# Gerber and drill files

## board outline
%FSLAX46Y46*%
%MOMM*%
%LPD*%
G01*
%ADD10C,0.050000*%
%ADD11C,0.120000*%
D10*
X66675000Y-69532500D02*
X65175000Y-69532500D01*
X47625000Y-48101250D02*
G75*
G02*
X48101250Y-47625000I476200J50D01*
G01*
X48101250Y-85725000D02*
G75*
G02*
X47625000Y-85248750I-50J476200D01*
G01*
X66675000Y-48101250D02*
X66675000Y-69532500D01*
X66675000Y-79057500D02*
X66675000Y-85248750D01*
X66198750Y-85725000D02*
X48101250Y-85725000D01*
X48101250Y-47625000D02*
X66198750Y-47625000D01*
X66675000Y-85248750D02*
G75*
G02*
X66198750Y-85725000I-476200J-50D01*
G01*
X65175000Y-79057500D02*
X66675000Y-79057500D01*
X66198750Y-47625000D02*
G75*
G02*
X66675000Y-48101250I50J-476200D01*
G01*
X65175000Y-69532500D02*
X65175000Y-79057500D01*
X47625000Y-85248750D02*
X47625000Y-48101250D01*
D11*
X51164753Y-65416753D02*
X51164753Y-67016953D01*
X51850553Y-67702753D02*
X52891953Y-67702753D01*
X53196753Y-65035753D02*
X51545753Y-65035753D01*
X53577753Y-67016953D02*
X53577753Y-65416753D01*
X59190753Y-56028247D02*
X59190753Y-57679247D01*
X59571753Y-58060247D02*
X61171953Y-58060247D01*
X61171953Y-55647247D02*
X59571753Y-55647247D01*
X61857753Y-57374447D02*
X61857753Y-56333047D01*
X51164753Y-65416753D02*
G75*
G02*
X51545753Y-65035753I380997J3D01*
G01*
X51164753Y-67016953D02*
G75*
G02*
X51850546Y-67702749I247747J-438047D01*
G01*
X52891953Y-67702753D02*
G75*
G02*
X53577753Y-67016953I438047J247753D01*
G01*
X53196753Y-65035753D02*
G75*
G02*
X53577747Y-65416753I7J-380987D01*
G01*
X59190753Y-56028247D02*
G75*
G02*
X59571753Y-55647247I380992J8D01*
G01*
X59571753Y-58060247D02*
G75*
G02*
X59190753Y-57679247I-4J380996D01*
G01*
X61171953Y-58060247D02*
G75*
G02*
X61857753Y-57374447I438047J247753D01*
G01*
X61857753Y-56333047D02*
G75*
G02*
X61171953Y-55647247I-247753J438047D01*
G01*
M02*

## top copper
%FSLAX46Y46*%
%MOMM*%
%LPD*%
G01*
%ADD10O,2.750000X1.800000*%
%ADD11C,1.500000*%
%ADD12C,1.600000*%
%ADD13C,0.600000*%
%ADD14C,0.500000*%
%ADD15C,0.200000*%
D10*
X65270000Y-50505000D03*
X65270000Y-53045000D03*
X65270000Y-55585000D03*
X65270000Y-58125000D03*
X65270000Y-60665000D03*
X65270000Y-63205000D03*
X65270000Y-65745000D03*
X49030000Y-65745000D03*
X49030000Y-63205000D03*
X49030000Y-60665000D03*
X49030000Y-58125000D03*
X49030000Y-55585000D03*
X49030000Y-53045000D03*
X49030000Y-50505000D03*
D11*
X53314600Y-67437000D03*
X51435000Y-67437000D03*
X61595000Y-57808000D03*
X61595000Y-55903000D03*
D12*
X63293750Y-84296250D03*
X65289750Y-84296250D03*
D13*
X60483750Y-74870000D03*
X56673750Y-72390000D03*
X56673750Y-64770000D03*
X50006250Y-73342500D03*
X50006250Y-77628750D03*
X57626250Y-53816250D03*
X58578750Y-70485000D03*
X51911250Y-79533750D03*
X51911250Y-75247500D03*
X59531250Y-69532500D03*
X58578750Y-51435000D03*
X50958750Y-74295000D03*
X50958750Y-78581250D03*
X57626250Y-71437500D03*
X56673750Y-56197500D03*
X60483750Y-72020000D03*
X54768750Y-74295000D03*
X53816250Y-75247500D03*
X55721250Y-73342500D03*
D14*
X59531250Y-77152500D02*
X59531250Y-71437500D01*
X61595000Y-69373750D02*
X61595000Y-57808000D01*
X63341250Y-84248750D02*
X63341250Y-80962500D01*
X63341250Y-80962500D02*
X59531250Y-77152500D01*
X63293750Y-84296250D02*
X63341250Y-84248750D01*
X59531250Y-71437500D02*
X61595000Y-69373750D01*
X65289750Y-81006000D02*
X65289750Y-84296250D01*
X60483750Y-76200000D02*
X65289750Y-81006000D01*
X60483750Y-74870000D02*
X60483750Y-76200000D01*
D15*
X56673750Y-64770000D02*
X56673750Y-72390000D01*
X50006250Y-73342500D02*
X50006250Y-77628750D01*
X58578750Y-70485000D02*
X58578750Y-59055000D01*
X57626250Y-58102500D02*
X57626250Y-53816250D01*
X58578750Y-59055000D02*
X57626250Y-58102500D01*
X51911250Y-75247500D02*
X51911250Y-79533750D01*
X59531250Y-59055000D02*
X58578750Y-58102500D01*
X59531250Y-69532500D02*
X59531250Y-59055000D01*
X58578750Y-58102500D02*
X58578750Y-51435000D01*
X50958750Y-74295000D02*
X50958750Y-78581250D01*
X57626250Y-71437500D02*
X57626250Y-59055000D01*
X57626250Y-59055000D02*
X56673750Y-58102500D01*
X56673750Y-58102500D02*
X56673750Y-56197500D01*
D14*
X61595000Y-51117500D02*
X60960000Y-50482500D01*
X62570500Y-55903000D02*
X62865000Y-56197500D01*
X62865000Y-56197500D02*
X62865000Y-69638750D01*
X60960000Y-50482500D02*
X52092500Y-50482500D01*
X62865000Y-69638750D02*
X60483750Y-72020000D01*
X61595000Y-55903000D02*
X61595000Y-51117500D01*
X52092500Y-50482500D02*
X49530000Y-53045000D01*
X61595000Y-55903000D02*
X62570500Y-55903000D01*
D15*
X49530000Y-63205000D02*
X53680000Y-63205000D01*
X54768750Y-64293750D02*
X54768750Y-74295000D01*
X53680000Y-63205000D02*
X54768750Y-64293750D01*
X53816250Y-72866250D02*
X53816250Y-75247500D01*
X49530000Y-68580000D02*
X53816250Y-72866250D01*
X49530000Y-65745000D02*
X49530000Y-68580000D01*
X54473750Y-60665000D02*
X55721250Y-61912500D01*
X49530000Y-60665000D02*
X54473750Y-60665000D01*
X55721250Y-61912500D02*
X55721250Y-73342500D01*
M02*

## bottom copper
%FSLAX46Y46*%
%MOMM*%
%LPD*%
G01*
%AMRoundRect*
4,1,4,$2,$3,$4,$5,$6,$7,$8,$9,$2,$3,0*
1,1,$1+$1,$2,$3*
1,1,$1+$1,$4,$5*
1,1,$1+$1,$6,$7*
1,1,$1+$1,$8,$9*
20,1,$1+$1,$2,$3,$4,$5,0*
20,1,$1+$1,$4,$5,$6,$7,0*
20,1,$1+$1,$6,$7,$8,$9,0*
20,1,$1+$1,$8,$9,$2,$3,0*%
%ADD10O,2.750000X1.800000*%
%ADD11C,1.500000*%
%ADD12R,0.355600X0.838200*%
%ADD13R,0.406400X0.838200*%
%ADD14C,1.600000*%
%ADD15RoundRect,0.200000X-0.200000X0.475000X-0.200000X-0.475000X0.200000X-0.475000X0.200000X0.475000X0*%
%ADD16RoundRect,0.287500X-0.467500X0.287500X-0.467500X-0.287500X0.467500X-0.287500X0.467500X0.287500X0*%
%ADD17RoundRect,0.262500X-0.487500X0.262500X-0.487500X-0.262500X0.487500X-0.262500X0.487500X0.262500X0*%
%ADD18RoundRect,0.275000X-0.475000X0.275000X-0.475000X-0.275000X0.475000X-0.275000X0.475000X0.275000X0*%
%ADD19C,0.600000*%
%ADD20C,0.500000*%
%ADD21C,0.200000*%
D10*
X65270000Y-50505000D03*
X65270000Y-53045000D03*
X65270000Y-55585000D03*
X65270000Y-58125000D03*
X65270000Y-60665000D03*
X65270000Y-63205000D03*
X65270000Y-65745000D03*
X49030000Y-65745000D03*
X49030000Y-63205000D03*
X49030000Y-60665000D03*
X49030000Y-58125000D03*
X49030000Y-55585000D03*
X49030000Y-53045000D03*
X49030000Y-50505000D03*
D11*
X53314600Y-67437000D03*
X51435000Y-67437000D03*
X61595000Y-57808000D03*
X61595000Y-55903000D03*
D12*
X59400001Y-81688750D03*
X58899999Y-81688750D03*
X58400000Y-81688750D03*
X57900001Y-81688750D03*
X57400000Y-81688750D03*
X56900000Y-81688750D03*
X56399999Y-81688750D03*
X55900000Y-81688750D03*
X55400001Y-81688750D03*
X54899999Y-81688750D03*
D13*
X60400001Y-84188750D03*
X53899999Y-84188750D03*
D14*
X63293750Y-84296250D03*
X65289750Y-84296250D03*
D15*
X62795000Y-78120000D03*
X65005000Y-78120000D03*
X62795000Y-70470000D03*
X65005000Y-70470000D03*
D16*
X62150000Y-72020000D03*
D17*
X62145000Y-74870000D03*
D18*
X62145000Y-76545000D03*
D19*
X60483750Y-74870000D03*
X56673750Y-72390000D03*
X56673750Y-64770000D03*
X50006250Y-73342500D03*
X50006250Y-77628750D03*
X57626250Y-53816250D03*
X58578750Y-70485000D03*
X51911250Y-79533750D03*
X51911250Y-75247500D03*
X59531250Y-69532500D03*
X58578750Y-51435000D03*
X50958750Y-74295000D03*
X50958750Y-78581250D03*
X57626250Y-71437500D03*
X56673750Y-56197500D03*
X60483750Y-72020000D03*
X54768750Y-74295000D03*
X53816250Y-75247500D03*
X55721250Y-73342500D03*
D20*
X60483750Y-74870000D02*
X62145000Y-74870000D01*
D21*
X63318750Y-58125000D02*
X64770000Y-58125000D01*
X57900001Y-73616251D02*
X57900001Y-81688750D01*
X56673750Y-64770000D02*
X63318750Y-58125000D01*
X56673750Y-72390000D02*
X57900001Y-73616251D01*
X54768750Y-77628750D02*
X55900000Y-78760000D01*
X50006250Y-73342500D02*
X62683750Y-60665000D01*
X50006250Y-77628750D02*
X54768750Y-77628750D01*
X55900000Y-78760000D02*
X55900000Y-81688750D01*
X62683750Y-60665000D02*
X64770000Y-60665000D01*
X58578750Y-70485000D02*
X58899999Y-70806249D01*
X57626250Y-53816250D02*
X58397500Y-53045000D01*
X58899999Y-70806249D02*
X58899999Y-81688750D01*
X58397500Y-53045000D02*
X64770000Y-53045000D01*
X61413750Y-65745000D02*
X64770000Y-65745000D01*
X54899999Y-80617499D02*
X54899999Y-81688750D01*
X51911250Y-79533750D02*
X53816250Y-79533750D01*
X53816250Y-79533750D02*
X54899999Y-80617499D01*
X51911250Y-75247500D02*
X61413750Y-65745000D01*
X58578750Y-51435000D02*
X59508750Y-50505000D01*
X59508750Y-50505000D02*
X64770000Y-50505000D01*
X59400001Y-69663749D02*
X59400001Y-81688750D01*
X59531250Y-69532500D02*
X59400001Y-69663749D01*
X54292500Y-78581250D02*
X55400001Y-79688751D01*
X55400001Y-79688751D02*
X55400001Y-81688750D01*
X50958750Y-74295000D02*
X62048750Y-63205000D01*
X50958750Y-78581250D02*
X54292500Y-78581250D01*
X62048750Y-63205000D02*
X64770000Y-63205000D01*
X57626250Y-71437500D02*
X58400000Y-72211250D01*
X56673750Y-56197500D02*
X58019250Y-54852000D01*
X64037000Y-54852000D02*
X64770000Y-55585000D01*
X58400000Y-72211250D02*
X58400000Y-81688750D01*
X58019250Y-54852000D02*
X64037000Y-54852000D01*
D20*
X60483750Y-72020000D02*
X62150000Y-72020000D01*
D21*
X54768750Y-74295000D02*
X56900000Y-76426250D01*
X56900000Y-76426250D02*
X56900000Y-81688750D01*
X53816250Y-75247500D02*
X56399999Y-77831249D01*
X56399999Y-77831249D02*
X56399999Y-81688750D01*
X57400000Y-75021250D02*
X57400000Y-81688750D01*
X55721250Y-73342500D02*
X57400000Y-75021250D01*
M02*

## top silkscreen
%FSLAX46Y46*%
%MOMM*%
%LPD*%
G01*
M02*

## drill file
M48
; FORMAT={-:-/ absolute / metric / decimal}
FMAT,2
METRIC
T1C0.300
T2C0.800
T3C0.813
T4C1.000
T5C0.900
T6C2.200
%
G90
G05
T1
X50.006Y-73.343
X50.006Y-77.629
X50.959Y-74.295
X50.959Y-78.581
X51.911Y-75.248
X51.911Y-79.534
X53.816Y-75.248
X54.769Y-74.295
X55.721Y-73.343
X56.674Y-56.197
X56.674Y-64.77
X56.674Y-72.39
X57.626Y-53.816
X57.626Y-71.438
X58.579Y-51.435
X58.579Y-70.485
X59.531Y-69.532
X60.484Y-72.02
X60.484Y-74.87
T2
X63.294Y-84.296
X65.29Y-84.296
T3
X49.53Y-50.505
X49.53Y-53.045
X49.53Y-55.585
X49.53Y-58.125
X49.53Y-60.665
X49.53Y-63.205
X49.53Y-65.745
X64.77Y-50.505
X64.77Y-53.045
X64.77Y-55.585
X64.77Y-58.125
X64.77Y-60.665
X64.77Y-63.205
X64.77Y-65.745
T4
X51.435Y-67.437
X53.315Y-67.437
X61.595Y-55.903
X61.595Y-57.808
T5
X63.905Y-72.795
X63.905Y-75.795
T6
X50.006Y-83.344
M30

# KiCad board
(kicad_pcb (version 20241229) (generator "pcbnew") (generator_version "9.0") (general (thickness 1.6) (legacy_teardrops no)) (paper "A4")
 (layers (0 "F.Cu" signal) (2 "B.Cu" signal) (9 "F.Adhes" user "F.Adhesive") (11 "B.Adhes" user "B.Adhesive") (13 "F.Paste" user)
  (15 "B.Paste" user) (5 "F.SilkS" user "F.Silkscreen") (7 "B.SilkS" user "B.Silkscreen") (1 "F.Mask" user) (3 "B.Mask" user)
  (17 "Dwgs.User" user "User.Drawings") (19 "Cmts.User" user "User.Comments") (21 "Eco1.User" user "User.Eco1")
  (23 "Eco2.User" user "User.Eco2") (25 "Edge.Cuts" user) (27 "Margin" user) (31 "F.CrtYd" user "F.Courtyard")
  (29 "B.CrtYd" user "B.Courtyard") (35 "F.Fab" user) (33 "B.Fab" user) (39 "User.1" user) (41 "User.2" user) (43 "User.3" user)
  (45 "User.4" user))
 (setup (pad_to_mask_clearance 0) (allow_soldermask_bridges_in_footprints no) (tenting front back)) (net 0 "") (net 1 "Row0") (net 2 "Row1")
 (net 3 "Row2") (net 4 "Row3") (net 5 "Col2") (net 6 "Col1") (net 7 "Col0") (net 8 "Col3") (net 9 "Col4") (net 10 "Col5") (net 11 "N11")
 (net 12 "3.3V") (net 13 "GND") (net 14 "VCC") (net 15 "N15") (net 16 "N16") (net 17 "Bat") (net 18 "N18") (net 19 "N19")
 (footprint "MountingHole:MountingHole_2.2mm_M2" (layer "F.Cu") (at 50.00625 83.34375)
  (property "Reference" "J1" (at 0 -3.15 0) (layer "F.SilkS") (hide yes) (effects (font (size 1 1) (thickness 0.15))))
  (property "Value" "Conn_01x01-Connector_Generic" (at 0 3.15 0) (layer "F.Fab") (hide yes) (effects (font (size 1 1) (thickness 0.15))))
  (pad "" np_thru_hole circle (at 0 0) (size 2.2 2.2) (drill 2.2) (layers "*.Cu" "*.Mask")))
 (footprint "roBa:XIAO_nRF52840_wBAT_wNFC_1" (layer "B.Cu") (at 57.15 47.625 180)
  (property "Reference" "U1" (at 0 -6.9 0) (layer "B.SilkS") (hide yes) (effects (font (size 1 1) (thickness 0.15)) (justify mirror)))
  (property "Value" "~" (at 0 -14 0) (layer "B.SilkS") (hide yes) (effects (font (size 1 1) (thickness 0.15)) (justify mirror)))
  (fp_line (start 5.985247 -17.791753) (end 5.985247 -19.391953) (stroke (width 0.12) (type solid)) (layer "Edge.Cuts"))
  (fp_line (start 5.299447 -20.077753) (end 4.258047 -20.077753) (stroke (width 0.12) (type solid)) (layer "Edge.Cuts"))
  (fp_line (start 3.953247 -17.410753) (end 5.604247 -17.410753) (stroke (width 0.12) (type solid)) (layer "Edge.Cuts"))
  (fp_line (start 3.572247 -19.391953) (end 3.572247 -17.791753) (stroke (width 0.12) (type solid)) (layer "Edge.Cuts"))
  (fp_line (start -2.040753 -8.403247) (end -2.040753 -10.054247) (stroke (width 0.12) (type solid)) (layer "Edge.Cuts"))
  (fp_line (start -2.421753 -10.435247) (end -4.021953 -10.435247) (stroke (width 0.12) (type solid)) (layer "Edge.Cuts"))
  (fp_line (start -4.021953 -8.022247) (end -2.421753 -8.022247) (stroke (width 0.12) (type solid)) (layer "Edge.Cuts"))
  (fp_line (start -4.707753 -9.749447) (end -4.707753 -8.708047) (stroke (width 0.12) (type solid)) (layer "Edge.Cuts"))
  (fp_arc (start 5.985247 -17.791753) (mid 5.873656 -17.522344) (end 5.604247 -17.410753) (stroke (width 0.12) (type solid))
   (layer "Edge.Cuts"))
  (fp_arc (start 5.985247 -19.391953) (mid 5.381645 -19.474147) (end 5.299447 -20.077753) (stroke (width 0.12) (type solid))
   (layer "Edge.Cuts"))
  (fp_arc (start 4.258047 -20.077753) (mid 4.175856 -19.474144) (end 3.572247 -19.391953) (stroke (width 0.12) (type solid))
   (layer "Edge.Cuts"))
  (fp_arc (start 3.953247 -17.410753) (mid 3.683836 -17.522343) (end 3.572247 -17.791753) (stroke (width 0.12) (type solid))
   (layer "Edge.Cuts"))
  (fp_arc (start -2.040753 -8.403247) (mid -2.152343 -8.133837) (end -2.421753 -8.022247) (stroke (width 0.12) (type solid))
   (layer "Edge.Cuts"))
  (fp_arc (start -2.421753 -10.435247) (mid -2.152344 -10.323656) (end -2.040753 -10.054247) (stroke (width 0.12) (type solid))
   (layer "Edge.Cuts"))
  (fp_arc (start -4.021953 -10.435247) (mid -4.104144 -9.831638) (end -4.707753 -9.749447) (stroke (width 0.12) (type solid))
   (layer "Edge.Cuts"))
  (fp_arc (start -4.707753 -8.708047) (mid -4.104144 -8.625856) (end -4.021953 -8.022247) (stroke (width 0.12) (type solid))
   (layer "Edge.Cuts"))
  (pad "1" thru_hole oval (at -7.62 -2.88 180) (size 2.75 1.8) (drill 0.8128 (offset -0.5 0)) (layers "*.Cu" "*.Mask")
   (remove_unused_layers no) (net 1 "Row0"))
  (pad "2" thru_hole oval (at -7.62 -5.42 180) (size 2.75 1.8) (drill 0.8128 (offset -0.5 0)) (layers "*.Cu" "*.Mask")
   (remove_unused_layers no) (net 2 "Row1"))
  (pad "3" thru_hole oval (at -7.62 -7.96 180) (size 2.75 1.8) (drill 0.8128 (offset -0.5 0)) (layers "*.Cu" "*.Mask")
   (remove_unused_layers no) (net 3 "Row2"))
  (pad "4" thru_hole oval (at -7.62 -10.5 180) (size 2.75 1.8) (drill 0.8128 (offset -0.5 0)) (layers "*.Cu" "*.Mask")
   (remove_unused_layers no) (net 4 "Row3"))
  (pad "5" thru_hole oval (at -7.62 -13.04 180) (size 2.75 1.8) (drill 0.8128 (offset -0.5 0)) (layers "*.Cu" "*.Mask")
   (remove_unused_layers no) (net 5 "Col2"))
  (pad "6" thru_hole oval (at -7.62 -15.58 180) (size 2.75 1.8) (drill 0.8128 (offset -0.5 0)) (layers "*.Cu" "*.Mask")
   (remove_unused_layers no) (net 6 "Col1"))
  (pad "7" thru_hole oval (at -7.62 -18.12 180) (size 2.75 1.8) (drill 0.8128 (offset -0.5 0)) (layers "*.Cu" "*.Mask")
   (remove_unused_layers no) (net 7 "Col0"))
  (pad "8" thru_hole oval (at 7.62 -18.12 180) (size 2.75 1.8) (drill 0.8128 (offset 0.5 0)) (layers "*.Cu" "*.Mask")
   (remove_unused_layers no) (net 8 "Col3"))
  (pad "9" thru_hole oval (at 7.62 -15.58 180) (size 2.75 1.8) (drill 0.8128 (offset 0.5 0)) (layers "*.Cu" "*.Mask")
   (remove_unused_layers no) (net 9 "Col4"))
  (pad "10" thru_hole oval (at 7.62 -13.04 180) (size 2.75 1.8) (drill 0.8128 (offset 0.5 0)) (layers "*.Cu" "*.Mask")
   (remove_unused_layers no) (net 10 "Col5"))
  (pad "11" thru_hole oval (at 7.62 -10.5 180) (size 2.75 1.8) (drill 0.8128 (offset 0.5 0)) (layers "*.Cu" "*.Mask")
   (remove_unused_layers no) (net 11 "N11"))
  (pad "12" thru_hole oval (at 7.62 -7.96 180) (size 2.75 1.8) (drill 0.8128 (offset 0.5 0)) (layers "*.Cu" "*.Mask")
   (remove_unused_layers no) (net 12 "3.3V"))
  (pad "13" thru_hole oval (at 7.62 -5.42 180) (size 2.75 1.8) (drill 0.8128 (offset 0.5 0)) (layers "*.Cu" "*.Mask")
   (remove_unused_layers no) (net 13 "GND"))
  (pad "14" thru_hole oval (at 7.62 -2.88 180) (size 2.75 1.8) (drill 0.8128 (offset 0.5 0)) (layers "*.Cu" "*.Mask")
   (remove_unused_layers no) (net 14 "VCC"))
  (pad "15" thru_hole circle (at 3.8354 -19.812 90) (size 1.5 1.5) (drill 1) (layers "*.Cu" "*.Mask") (remove_unused_layers no)
   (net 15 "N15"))
  (pad "16" thru_hole circle (at 5.715 -19.812 270) (size 1.5 1.5) (drill 1) (layers "*.Cu" "*.Mask") (remove_unused_layers no)
   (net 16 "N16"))
  (pad "20" thru_hole circle (at -4.445 -10.183 270) (size 1.5 1.5) (drill 1) (layers "*.Cu" "*.Mask") (remove_unused_layers no)
   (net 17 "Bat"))
  (pad "21" thru_hole circle (at -4.445 -8.278 90) (size 1.5 1.5) (drill 1) (layers "*.Cu" "*.Mask") (remove_unused_layers no)
   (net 13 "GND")))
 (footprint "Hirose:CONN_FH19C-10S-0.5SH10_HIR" (layer "B.Cu") (at 57.15 83.34375 180)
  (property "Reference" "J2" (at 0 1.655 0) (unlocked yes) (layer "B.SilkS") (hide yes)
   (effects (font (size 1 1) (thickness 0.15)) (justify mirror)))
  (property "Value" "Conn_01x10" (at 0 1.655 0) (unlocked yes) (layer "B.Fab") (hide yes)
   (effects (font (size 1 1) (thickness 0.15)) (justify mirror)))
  (pad "1" smd rect (at -2.250001 1.655 180) (size 0.3556 0.8382) (layers "B.Cu" "B.Mask" "B.Paste") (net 1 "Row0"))
  (pad "2" smd rect (at -1.749999 1.655 180) (size 0.3556 0.8382) (layers "B.Cu" "B.Mask" "B.Paste") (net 2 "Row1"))
  (pad "3" smd rect (at -1.25 1.655 180) (size 0.3556 0.8382) (layers "B.Cu" "B.Mask" "B.Paste") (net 3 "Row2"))
  (pad "4" smd rect (at -0.750001 1.655 180) (size 0.3556 0.8382) (layers "B.Cu" "B.Mask" "B.Paste") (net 4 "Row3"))
  (pad "5" smd rect (at -0.25 1.655 180) (size 0.3556 0.8382) (layers "B.Cu" "B.Mask" "B.Paste") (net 10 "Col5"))
  (pad "6" smd rect (at 0.25 1.655 180) (size 0.3556 0.8382) (layers "B.Cu" "B.Mask" "B.Paste") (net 9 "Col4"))
  (pad "7" smd rect (at 0.750001 1.655 180) (size 0.3556 0.8382) (layers "B.Cu" "B.Mask" "B.Paste") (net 8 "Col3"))
  (pad "8" smd rect (at 1.25 1.655 180) (size 0.3556 0.8382) (layers "B.Cu" "B.Mask" "B.Paste") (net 5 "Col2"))
  (pad "9" smd rect (at 1.749999 1.655 180) (size 0.3556 0.8382) (layers "B.Cu" "B.Mask" "B.Paste") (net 6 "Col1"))
  (pad "10" smd rect (at 2.250001 1.655 180) (size 0.3556 0.8382) (layers "B.Cu" "B.Mask" "B.Paste") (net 7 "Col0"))
  (pad "11" smd rect (at -3.250001 -0.845 180) (size 0.4064 0.8382) (layers "B.Cu" "B.Mask" "B.Paste"))
  (pad "12" smd rect (at 3.250001 -0.845 180) (size 0.4064 0.8382) (layers "B.Cu" "B.Mask" "B.Paste")))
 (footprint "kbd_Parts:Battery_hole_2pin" (layer "B.Cu") (at 64.29375 84.29625 -90)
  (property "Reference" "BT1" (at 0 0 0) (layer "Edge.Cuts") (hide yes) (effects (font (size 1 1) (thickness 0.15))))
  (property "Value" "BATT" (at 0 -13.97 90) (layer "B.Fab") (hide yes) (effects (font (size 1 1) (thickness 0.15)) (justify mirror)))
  (pad "1" thru_hole circle (at 0 1 270) (size 1.6 1.6) (drill 0.8) (layers "*.Cu" "*.Mask" "B.SilkS") (remove_unused_layers no)
   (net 17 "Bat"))
  (pad "2" thru_hole circle (at 0 -0.996 270) (size 1.6 1.6) (drill 0.8) (layers "*.Cu" "*.Mask" "B.SilkS") (remove_unused_layers no)
   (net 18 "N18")))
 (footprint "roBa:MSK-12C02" (layer "B.Cu") (at 63.905 74.295 90)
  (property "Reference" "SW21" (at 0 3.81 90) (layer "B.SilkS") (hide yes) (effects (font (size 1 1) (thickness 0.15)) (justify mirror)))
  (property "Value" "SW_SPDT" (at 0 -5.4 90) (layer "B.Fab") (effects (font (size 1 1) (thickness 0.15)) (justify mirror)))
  (pad "" smd roundrect (at -3.825 -1.11 270) (size 1.35 0.8) (layers "B.Cu" "B.Mask" "B.Paste") (roundrect_rratio 0.25))
  (pad "" smd roundrect (at -3.825 1.1 270) (size 1.35 0.8) (layers "B.Cu" "B.Mask" "B.Paste") (roundrect_rratio 0.25))
  (pad "" np_thru_hole circle (at -1.5 0 270) (size 0.9 0.9) (drill 0.9) (layers "*.Cu" "*.Mask"))
  (pad "" np_thru_hole circle (at 1.5 0 270) (size 0.9 0.9) (drill 0.9) (layers "*.Cu" "*.Mask"))
  (pad "" smd roundrect (at 3.825 -1.11 270) (size 1.35 0.8) (layers "B.Cu" "B.Mask" "B.Paste") (roundrect_rratio 0.25))
  (pad "" smd roundrect (at 3.825 1.1 270) (size 1.35 0.8) (layers "B.Cu" "B.Mask" "B.Paste") (roundrect_rratio 0.25))
  (pad "1" smd roundrect (at 2.275 -1.755 270) (size 1.15 1.51) (layers "B.Cu" "B.Mask" "B.Paste") (roundrect_rratio 0.25) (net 13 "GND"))
  (pad "2" smd roundrect (at -0.575 -1.76 270) (size 1.05 1.5) (layers "B.Cu" "B.Mask" "B.Paste") (roundrect_rratio 0.25) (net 18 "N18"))
  (pad "3" smd roundrect (at -2.25 -1.76 270) (size 1.1 1.5) (layers "B.Cu" "B.Mask" "B.Paste") (roundrect_rratio 0.25) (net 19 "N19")))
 (gr_line (start 66.675 69.5325) (end 65.175 69.5325) (stroke (width 0.05) (type default)) (layer "Edge.Cuts"))
 (gr_arc (start 47.625 48.10125) (mid 47.76449 47.76449) (end 48.10125 47.625) (stroke (width 0.05) (type default)) (layer "Edge.Cuts"))
 (gr_arc (start 48.10125 85.725) (mid 47.76449 85.58551) (end 47.625 85.24875) (stroke (width 0.05) (type default)) (layer "Edge.Cuts"))
 (gr_line (start 66.675 48.10125) (end 66.675 69.5325) (stroke (width 0.05) (type default)) (layer "Edge.Cuts"))
 (gr_line (start 66.675 79.0575) (end 66.675 85.24875) (stroke (width 0.05) (type default)) (layer "Edge.Cuts"))
 (gr_line (start 66.19875 85.725) (end 48.10125 85.725) (stroke (width 0.05) (type default)) (layer "Edge.Cuts"))
 (gr_line (start 48.10125 47.625) (end 66.19875 47.625) (stroke (width 0.05) (type default)) (layer "Edge.Cuts"))
 (gr_arc (start 66.675 85.24875) (mid 66.53551 85.58551) (end 66.19875 85.725) (stroke (width 0.05) (type default)) (layer "Edge.Cuts"))
 (gr_line (start 65.175 79.0575) (end 66.675 79.0575) (stroke (width 0.05) (type default)) (layer "Edge.Cuts"))
 (gr_arc (start 66.19875 47.625) (mid 66.53551 47.76449) (end 66.675 48.10125) (stroke (width 0.05) (type default)) (layer "Edge.Cuts"))
 (gr_line (start 65.175 69.5325) (end 65.175 79.0575) (stroke (width 0.05) (type solid)) (layer "Edge.Cuts"))
 (gr_line (start 47.625 85.24875) (end 47.625 48.10125) (stroke (width 0.05) (type default)) (layer "Edge.Cuts"))
 (segment (start 59.53125 77.1525) (end 59.53125 71.4375) (width 0.5) (layer "F.Cu") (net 17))
 (segment (start 61.595 69.37375) (end 61.595 57.808) (width 0.5) (layer "F.Cu") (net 17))
 (segment (start 63.34125 84.24875) (end 63.34125 80.9625) (width 0.5) (layer "F.Cu") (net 17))
 (segment (start 63.34125 80.9625) (end 59.53125 77.1525) (width 0.5) (layer "F.Cu") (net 17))
 (segment (start 63.29375 84.29625) (end 63.34125 84.24875) (width 0.5) (layer "F.Cu") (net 17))
 (segment (start 59.53125 71.4375) (end 61.595 69.37375) (width 0.5) (layer "F.Cu") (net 17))
 (segment (start 65.28975 81.006) (end 65.28975 84.29625) (width 0.5) (layer "F.Cu") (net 18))
 (segment (start 60.48375 76.2) (end 65.28975 81.006) (width 0.5) (layer "F.Cu") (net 18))
 (segment (start 60.48375 74.87) (end 60.48375 76.2) (width 0.5) (layer "F.Cu") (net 18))
 (via (at 60.48375 74.87) (size 0.6) (drill 0.3) (layers "F.Cu" "B.Cu") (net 18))
 (segment (start 60.48375 74.87) (end 62.145 74.87) (width 0.5) (layer "B.Cu") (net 18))
 (segment (start 56.67375 64.77) (end 56.67375 72.39) (width 0.2) (layer "F.Cu") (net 4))
 (via (at 56.67375 72.39) (size 0.6) (drill 0.3) (layers "F.Cu" "B.Cu") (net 4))
 (via (at 56.67375 64.77) (size 0.6) (drill 0.3) (layers "F.Cu" "B.Cu") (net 4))
 (segment (start 63.31875 58.125) (end 64.77 58.125) (width 0.2) (layer "B.Cu") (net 4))
 (segment (start 57.900001 73.616251) (end 57.900001 81.68875) (width 0.2) (layer "B.Cu") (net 4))
 (segment (start 56.67375 64.77) (end 63.31875 58.125) (width 0.2) (layer "B.Cu") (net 4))
 (segment (start 56.67375 72.39) (end 57.900001 73.616251) (width 0.2) (layer "B.Cu") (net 4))
 (segment (start 50.00625 73.3425) (end 50.00625 77.62875) (width 0.2) (layer "F.Cu") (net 5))
 (via (at 50.00625 73.3425) (size 0.6) (drill 0.3) (layers "F.Cu" "B.Cu") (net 5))
 (via (at 50.00625 77.62875) (size 0.6) (drill 0.3) (layers "F.Cu" "B.Cu") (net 5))
 (segment (start 54.76875 77.62875) (end 55.9 78.76) (width 0.2) (layer "B.Cu") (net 5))
 (segment (start 50.00625 73.3425) (end 62.68375 60.665) (width 0.2) (layer "B.Cu") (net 5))
 (segment (start 50.00625 77.62875) (end 54.76875 77.62875) (width 0.2) (layer "B.Cu") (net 5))
 (segment (start 55.9 78.76) (end 55.9 81.68875) (width 0.2) (layer "B.Cu") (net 5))
 (segment (start 62.68375 60.665) (end 64.77 60.665) (width 0.2) (layer "B.Cu") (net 5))
 (segment (start 58.57875 70.485) (end 58.57875 59.055) (width 0.2) (layer "F.Cu") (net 2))
 (segment (start 57.62625 58.1025) (end 57.62625 53.81625) (width 0.2) (layer "F.Cu") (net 2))
 (segment (start 58.57875 59.055) (end 57.62625 58.1025) (width 0.2) (layer "F.Cu") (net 2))
 (via (at 57.62625 53.81625) (size 0.6) (drill 0.3) (layers "F.Cu" "B.Cu") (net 2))
 (via (at 58.57875 70.485) (size 0.6) (drill 0.3) (layers "F.Cu" "B.Cu") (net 2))
 (segment (start 58.57875 70.485) (end 58.899999 70.806249) (width 0.2) (layer "B.Cu") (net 2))
 (segment (start 57.62625 53.81625) (end 58.3975 53.045) (width 0.2) (layer "B.Cu") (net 2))
 (segment (start 58.899999 70.806249) (end 58.899999 81.68875) (width 0.2) (layer "B.Cu") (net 2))
 (segment (start 58.3975 53.045) (end 64.77 53.045) (width 0.2) (layer "B.Cu") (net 2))
 (segment (start 51.91125 75.2475) (end 51.91125 79.53375) (width 0.2) (layer "F.Cu") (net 7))
 (via (at 51.91125 79.53375) (size 0.6) (drill 0.3) (layers "F.Cu" "B.Cu") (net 7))
 (via (at 51.91125 75.2475) (size 0.6) (drill 0.3) (layers "F.Cu" "B.Cu") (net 7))
 (segment (start 61.41375 65.745) (end 64.77 65.745) (width 0.2) (layer "B.Cu") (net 7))
 (segment (start 54.899999 80.617499) (end 54.899999 81.68875) (width 0.2) (layer "B.Cu") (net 7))
 (segment (start 51.91125 79.53375) (end 53.81625 79.53375) (width 0.2) (layer "B.Cu") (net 7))
 (segment (start 53.81625 79.53375) (end 54.899999 80.617499) (width 0.2) (layer "B.Cu") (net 7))
 (segment (start 51.91125 75.2475) (end 61.41375 65.745) (width 0.2) (layer "B.Cu") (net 7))
 (segment (start 59.53125 59.055) (end 58.57875 58.1025) (width 0.2) (layer "F.Cu") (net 1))
 (segment (start 59.53125 69.5325) (end 59.53125 59.055) (width 0.2) (layer "F.Cu") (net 1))
 (segment (start 58.57875 58.1025) (end 58.57875 51.435) (width 0.2) (layer "F.Cu") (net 1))
 (via (at 59.53125 69.5325) (size 0.6) (drill 0.3) (layers "F.Cu" "B.Cu") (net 1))
 (via (at 58.57875 51.435) (size 0.6) (drill 0.3) (layers "F.Cu" "B.Cu") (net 1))
 (segment (start 58.57875 51.435) (end 59.50875 50.505) (width 0.2) (layer "B.Cu") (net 1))
 (segment (start 59.50875 50.505) (end 64.77 50.505) (width 0.2) (layer "B.Cu") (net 1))
 (segment (start 59.400001 69.663749) (end 59.400001 81.68875) (width 0.2) (layer "B.Cu") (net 1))
 (segment (start 59.53125 69.5325) (end 59.400001 69.663749) (width 0.2) (layer "B.Cu") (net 1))
 (segment (start 50.95875 74.295) (end 50.95875 78.58125) (width 0.2) (layer "F.Cu") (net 6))
 (via (at 50.95875 74.295) (size 0.6) (drill 0.3) (layers "F.Cu" "B.Cu") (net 6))
 (via (at 50.95875 78.58125) (size 0.6) (drill 0.3) (layers "F.Cu" "B.Cu") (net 6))
 (segment (start 54.2925 78.58125) (end 55.400001 79.688751) (width 0.2) (layer "B.Cu") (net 6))
 (segment (start 55.400001 79.688751) (end 55.400001 81.68875) (width 0.2) (layer "B.Cu") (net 6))
 (segment (start 50.95875 74.295) (end 62.04875 63.205) (width 0.2) (layer "B.Cu") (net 6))
 (segment (start 50.95875 78.58125) (end 54.2925 78.58125) (width 0.2) (layer "B.Cu") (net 6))
 (segment (start 62.04875 63.205) (end 64.77 63.205) (width 0.2) (layer "B.Cu") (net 6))
 (segment (start 57.62625 71.4375) (end 57.62625 59.055) (width 0.2) (layer "F.Cu") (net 3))
 (segment (start 57.62625 59.055) (end 56.67375 58.1025) (width 0.2) (layer "F.Cu") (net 3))
 (segment (start 56.67375 58.1025) (end 56.67375 56.1975) (width 0.2) (layer "F.Cu") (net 3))
 (via (at 57.62625 71.4375) (size 0.6) (drill 0.3) (layers "F.Cu" "B.Cu") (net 3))
 (via (at 56.67375 56.1975) (size 0.6) (drill 0.3) (layers "F.Cu" "B.Cu") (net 3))
 (segment (start 57.62625 71.4375) (end 58.4 72.21125) (width 0.2) (layer "B.Cu") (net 3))
 (segment (start 56.67375 56.1975) (end 58.01925 54.852) (width 0.2) (layer "B.Cu") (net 3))
 (segment (start 64.037 54.852) (end 64.77 55.585) (width 0.2) (layer "B.Cu") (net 3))
 (segment (start 58.4 72.21125) (end 58.4 81.68875) (width 0.2) (layer "B.Cu") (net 3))
 (segment (start 58.01925 54.852) (end 64.037 54.852) (width 0.2) (layer "B.Cu") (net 3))
 (segment (start 61.595 51.1175) (end 60.96 50.4825) (width 0.5) (layer "F.Cu") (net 13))
 (segment (start 62.5705 55.903) (end 62.865 56.1975) (width 0.5) (layer "F.Cu") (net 13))
 (segment (start 62.865 56.1975) (end 62.865 69.63875) (width 0.5) (layer "F.Cu") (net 13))
 (segment (start 60.96 50.4825) (end 52.0925 50.4825) (width 0.5) (layer "F.Cu") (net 13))
 (segment (start 62.865 69.63875) (end 60.48375 72.02) (width 0.5) (layer "F.Cu") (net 13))
 (segment (start 61.595 55.903) (end 61.595 51.1175) (width 0.5) (layer "F.Cu") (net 13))
 (segment (start 52.0925 50.4825) (end 49.53 53.045) (width 0.5) (layer "F.Cu") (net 13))
 (segment (start 61.595 55.903) (end 62.5705 55.903) (width 0.5) (layer "F.Cu") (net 13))
 (via (at 60.48375 72.02) (size 0.6) (drill 0.3) (layers "F.Cu" "B.Cu") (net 13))
 (segment (start 60.48375 72.02) (end 62.15 72.02) (width 0.5) (layer "B.Cu") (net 13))
 (segment (start 49.53 63.205) (end 53.68 63.205) (width 0.2) (layer "F.Cu") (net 9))
 (segment (start 54.76875 64.29375) (end 54.76875 74.295) (width 0.2) (layer "F.Cu") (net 9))
 (segment (start 53.68 63.205) (end 54.76875 64.29375) (width 0.2) (layer "F.Cu") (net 9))
 (via (at 54.76875 74.295) (size 0.6) (drill 0.3) (layers "F.Cu" "B.Cu") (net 9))
 (segment (start 54.76875 74.295) (end 56.9 76.42625) (width 0.2) (layer "B.Cu") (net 9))
 (segment (start 56.9 76.42625) (end 56.9 81.68875) (width 0.2) (layer "B.Cu") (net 9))
 (segment (start 53.81625 72.86625) (end 53.81625 75.2475) (width 0.2) (layer "F.Cu") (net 8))
 (segment (start 49.53 68.58) (end 53.81625 72.86625) (width 0.2) (layer "F.Cu") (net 8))
 (segment (start 49.53 65.745) (end 49.53 68.58) (width 0.2) (layer "F.Cu") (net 8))
 (via (at 53.81625 75.2475) (size 0.6) (drill 0.3) (layers "F.Cu" "B.Cu") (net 8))
 (segment (start 53.81625 75.2475) (end 56.399999 77.831249) (width 0.2) (layer "B.Cu") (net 8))
 (segment (start 56.399999 77.831249) (end 56.399999 81.68875) (width 0.2) (layer "B.Cu") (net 8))
 (segment (start 54.47375 60.665) (end 55.72125 61.9125) (width 0.2) (layer "F.Cu") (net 10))
 (segment (start 49.53 60.665) (end 54.47375 60.665) (width 0.2) (layer "F.Cu") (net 10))
 (segment (start 55.72125 61.9125) (end 55.72125 73.3425) (width 0.2) (layer "F.Cu") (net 10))
 (via (at 55.72125 73.3425) (size 0.6) (drill 0.3) (layers "F.Cu" "B.Cu") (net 10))
 (segment (start 57.4 75.02125) (end 57.4 81.68875) (width 0.2) (layer "B.Cu") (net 10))
 (segment (start 55.72125 73.3425) (end 57.4 75.02125) (width 0.2) (layer "B.Cu") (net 10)))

